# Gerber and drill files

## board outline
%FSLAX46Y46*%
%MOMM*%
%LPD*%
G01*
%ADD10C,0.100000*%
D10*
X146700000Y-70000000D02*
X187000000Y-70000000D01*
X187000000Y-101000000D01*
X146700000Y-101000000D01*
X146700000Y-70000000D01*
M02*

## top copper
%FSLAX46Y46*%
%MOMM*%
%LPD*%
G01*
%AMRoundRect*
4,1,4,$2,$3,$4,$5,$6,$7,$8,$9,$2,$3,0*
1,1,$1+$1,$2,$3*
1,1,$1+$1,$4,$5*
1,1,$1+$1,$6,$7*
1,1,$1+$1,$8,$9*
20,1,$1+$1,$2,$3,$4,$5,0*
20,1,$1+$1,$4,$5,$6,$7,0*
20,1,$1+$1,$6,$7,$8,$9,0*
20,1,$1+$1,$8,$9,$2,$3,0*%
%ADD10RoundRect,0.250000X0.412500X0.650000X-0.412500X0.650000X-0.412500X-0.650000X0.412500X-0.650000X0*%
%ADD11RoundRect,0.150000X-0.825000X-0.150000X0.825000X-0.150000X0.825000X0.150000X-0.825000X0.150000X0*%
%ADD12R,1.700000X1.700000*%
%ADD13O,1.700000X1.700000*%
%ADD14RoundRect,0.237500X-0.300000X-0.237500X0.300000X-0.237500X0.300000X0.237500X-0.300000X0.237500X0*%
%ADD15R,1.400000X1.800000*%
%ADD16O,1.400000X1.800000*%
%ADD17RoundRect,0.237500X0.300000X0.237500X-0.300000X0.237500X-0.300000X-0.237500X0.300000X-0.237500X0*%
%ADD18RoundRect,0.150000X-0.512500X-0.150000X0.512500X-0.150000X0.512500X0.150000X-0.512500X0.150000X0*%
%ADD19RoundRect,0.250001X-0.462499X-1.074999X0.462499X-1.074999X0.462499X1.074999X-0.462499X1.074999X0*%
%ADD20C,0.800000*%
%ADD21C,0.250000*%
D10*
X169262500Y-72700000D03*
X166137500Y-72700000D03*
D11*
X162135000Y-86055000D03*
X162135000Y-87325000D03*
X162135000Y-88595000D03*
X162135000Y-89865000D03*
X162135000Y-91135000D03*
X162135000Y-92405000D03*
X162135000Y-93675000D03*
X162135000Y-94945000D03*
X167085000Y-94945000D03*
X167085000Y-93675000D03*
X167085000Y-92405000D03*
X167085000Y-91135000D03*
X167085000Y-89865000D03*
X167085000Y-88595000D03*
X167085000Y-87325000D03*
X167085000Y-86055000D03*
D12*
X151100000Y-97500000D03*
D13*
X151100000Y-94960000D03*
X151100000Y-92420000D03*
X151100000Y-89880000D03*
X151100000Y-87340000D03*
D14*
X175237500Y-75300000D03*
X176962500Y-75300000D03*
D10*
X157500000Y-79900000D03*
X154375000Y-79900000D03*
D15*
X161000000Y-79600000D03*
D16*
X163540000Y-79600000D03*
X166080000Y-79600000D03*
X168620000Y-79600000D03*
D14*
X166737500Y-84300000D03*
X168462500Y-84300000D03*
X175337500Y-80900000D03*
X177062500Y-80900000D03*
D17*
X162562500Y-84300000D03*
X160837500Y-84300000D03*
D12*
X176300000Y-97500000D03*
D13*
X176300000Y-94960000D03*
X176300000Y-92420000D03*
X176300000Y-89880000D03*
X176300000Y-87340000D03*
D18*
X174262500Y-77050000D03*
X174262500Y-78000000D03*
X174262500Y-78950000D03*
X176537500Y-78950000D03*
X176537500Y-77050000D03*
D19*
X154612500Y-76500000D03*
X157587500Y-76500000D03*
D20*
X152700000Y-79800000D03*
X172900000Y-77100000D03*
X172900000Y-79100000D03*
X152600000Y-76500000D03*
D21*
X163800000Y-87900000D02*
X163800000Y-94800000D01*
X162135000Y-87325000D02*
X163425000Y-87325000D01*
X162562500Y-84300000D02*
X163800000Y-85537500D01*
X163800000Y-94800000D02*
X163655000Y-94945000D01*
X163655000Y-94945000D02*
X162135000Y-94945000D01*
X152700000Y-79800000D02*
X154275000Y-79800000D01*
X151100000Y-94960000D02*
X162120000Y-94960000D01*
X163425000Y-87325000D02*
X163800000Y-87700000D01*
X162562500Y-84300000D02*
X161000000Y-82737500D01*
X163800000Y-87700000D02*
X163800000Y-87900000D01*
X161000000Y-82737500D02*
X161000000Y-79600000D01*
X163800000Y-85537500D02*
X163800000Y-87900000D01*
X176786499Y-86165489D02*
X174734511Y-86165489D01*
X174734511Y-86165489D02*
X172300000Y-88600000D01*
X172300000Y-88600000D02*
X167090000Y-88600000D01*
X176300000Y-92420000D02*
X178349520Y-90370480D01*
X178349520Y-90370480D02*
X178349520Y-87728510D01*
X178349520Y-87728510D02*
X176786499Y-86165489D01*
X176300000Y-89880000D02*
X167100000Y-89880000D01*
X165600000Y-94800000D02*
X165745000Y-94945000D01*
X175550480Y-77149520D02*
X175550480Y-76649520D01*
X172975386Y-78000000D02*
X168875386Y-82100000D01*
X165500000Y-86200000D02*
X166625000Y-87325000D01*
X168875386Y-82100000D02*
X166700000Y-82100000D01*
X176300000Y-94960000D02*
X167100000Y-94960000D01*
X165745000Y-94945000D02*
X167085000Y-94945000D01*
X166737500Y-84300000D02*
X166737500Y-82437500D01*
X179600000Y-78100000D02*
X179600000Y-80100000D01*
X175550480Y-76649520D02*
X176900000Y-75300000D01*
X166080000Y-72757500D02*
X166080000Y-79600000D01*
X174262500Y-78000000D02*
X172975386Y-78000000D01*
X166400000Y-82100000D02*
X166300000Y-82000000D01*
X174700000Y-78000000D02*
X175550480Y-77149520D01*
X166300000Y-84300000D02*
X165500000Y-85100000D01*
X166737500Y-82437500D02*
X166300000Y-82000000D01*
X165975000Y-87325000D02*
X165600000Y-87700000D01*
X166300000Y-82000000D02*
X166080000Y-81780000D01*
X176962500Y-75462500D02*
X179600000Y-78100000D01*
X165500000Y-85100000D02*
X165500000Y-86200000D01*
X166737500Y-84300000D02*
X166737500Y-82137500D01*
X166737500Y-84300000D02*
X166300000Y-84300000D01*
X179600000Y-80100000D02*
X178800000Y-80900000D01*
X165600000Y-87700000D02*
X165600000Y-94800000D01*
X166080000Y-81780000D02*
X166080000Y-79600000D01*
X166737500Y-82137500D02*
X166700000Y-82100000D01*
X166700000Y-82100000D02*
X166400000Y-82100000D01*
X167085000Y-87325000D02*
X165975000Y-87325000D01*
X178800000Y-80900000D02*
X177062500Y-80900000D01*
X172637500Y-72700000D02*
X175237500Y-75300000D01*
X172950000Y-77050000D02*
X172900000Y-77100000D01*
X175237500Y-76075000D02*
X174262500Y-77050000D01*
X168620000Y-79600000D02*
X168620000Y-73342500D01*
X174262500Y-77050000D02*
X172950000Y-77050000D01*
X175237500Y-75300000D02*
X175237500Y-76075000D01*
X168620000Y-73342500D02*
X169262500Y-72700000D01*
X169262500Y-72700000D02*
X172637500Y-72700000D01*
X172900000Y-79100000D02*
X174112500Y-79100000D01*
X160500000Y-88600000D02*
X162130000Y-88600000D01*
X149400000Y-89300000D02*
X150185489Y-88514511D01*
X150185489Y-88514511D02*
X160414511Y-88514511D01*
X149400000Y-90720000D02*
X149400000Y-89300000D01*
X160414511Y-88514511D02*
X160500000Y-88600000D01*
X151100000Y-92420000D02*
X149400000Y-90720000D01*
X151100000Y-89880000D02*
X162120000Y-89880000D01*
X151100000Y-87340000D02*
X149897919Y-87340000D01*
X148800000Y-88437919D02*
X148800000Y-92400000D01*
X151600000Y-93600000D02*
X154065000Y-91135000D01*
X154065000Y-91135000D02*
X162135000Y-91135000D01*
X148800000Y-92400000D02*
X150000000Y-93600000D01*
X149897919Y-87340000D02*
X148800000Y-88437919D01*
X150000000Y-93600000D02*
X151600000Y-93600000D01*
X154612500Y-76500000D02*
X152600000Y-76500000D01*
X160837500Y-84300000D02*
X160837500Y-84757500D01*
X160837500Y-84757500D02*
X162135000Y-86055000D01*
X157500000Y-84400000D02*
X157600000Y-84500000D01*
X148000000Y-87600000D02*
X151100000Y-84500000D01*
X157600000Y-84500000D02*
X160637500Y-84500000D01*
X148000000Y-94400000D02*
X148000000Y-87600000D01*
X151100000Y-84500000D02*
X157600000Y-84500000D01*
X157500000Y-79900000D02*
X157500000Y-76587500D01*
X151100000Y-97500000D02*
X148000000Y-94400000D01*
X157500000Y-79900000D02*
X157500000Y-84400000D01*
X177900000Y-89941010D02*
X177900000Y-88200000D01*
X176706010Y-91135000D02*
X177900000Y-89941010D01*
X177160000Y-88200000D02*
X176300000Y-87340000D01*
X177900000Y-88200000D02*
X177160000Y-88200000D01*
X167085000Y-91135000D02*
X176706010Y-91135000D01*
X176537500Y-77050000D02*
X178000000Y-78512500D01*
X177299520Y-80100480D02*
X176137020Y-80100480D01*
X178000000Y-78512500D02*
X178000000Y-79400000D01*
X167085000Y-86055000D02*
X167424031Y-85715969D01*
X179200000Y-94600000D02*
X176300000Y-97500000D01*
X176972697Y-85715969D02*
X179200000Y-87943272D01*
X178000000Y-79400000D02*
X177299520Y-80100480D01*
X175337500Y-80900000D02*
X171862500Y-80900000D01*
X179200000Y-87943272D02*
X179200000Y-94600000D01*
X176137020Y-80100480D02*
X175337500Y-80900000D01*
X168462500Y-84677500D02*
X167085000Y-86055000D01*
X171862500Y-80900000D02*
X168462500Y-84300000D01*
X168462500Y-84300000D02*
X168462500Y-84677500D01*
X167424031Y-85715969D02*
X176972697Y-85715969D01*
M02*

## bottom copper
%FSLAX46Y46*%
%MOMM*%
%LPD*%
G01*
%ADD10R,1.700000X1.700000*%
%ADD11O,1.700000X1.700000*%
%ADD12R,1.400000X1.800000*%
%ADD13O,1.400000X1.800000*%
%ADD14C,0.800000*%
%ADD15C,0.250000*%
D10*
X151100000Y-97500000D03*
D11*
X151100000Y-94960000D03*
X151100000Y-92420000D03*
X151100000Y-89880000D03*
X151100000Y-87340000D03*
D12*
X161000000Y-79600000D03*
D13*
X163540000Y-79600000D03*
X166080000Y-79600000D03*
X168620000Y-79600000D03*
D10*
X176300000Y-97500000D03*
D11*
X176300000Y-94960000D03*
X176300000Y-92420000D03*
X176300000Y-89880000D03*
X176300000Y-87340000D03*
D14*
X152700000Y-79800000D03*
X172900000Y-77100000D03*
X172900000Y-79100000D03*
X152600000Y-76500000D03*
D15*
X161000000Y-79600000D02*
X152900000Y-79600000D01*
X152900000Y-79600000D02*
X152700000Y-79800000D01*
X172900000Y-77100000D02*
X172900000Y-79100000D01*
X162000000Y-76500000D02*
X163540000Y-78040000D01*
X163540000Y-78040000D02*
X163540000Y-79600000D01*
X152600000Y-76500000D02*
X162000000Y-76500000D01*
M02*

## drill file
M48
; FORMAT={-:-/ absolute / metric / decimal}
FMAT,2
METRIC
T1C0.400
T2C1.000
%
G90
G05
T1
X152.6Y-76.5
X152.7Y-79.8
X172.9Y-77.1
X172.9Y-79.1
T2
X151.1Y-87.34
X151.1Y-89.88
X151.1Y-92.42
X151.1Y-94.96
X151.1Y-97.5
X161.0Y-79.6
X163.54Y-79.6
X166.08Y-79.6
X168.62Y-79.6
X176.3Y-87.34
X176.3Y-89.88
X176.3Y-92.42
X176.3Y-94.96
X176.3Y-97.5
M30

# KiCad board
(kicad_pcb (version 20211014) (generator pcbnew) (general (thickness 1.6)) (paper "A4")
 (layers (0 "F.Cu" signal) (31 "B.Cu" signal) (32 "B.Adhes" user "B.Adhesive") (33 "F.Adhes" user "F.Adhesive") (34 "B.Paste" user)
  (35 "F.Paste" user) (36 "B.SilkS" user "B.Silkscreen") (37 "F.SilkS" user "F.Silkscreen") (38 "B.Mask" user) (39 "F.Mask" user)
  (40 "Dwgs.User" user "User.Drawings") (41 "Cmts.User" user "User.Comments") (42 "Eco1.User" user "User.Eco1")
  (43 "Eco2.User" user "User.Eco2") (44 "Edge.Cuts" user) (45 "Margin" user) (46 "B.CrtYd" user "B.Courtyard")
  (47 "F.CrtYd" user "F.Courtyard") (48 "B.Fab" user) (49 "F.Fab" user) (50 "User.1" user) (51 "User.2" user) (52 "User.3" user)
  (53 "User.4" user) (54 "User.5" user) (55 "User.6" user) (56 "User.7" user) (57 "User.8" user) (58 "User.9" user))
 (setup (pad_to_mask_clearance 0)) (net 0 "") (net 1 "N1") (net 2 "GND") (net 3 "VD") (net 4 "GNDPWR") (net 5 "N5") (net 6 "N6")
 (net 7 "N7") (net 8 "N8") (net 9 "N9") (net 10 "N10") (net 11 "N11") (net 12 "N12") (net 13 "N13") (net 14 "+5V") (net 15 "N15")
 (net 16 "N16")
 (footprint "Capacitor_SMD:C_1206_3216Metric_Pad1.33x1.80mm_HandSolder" (layer "F.Cu") (at 167.7 72.7 180)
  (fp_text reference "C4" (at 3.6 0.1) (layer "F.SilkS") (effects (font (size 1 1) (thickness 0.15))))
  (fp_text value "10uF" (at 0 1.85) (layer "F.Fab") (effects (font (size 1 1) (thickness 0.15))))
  (pad "1" smd roundrect (at -1.5625 0 180) (size 1.325 1.8) (layers "F.Cu" "F.Paste" "F.Mask") (roundrect_rratio 0.1886792453) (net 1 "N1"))
  (pad "2" smd roundrect (at 1.5625 0 180) (size 1.325 1.8) (layers "F.Cu" "F.Paste" "F.Mask") (roundrect_rratio 0.1886792453) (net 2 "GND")))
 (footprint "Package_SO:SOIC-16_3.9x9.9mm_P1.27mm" (layer "F.Cu") (at 164.61 90.5)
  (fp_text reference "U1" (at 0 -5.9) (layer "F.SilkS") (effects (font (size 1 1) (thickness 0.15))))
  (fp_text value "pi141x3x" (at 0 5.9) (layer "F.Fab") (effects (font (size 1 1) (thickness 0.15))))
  (pad "1" smd roundrect (at -2.475 -4.445) (size 1.95 0.6) (layers "F.Cu" "F.Paste" "F.Mask") (roundrect_rratio 0.25) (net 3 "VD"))
  (pad "2" smd roundrect (at -2.475 -3.175) (size 1.95 0.6) (layers "F.Cu" "F.Paste" "F.Mask") (roundrect_rratio 0.25) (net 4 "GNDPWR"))
  (pad "3" smd roundrect (at -2.475 -1.905) (size 1.95 0.6) (layers "F.Cu" "F.Paste" "F.Mask") (roundrect_rratio 0.25) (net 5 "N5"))
  (pad "4" smd roundrect (at -2.475 -0.635) (size 1.95 0.6) (layers "F.Cu" "F.Paste" "F.Mask") (roundrect_rratio 0.25) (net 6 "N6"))
  (pad "5" smd roundrect (at -2.475 0.635) (size 1.95 0.6) (layers "F.Cu" "F.Paste" "F.Mask") (roundrect_rratio 0.25) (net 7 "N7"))
  (pad "6" smd roundrect (at -2.475 1.905) (size 1.95 0.6) (layers "F.Cu" "F.Paste" "F.Mask") (roundrect_rratio 0.25) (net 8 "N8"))
  (pad "7" smd roundrect (at -2.475 3.175) (size 1.95 0.6) (layers "F.Cu" "F.Paste" "F.Mask") (roundrect_rratio 0.25) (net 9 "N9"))
  (pad "8" smd roundrect (at -2.475 4.445) (size 1.95 0.6) (layers "F.Cu" "F.Paste" "F.Mask") (roundrect_rratio 0.25) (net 4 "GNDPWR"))
  (pad "9" smd roundrect (at 2.475 4.445) (size 1.95 0.6) (layers "F.Cu" "F.Paste" "F.Mask") (roundrect_rratio 0.25) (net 2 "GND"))
  (pad "10" smd roundrect (at 2.475 3.175) (size 1.95 0.6) (layers "F.Cu" "F.Paste" "F.Mask") (roundrect_rratio 0.25) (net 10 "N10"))
  (pad "11" smd roundrect (at 2.475 1.905) (size 1.95 0.6) (layers "F.Cu" "F.Paste" "F.Mask") (roundrect_rratio 0.25) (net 2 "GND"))
  (pad "12" smd roundrect (at 2.475 0.635) (size 1.95 0.6) (layers "F.Cu" "F.Paste" "F.Mask") (roundrect_rratio 0.25) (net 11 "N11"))
  (pad "13" smd roundrect (at 2.475 -0.635) (size 1.95 0.6) (layers "F.Cu" "F.Paste" "F.Mask") (roundrect_rratio 0.25) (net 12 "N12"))
  (pad "14" smd roundrect (at 2.475 -1.905) (size 1.95 0.6) (layers "F.Cu" "F.Paste" "F.Mask") (roundrect_rratio 0.25) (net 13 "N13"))
  (pad "15" smd roundrect (at 2.475 -3.175) (size 1.95 0.6) (layers "F.Cu" "F.Paste" "F.Mask") (roundrect_rratio 0.25) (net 2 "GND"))
  (pad "16" smd roundrect (at 2.475 -4.445) (size 1.95 0.6) (layers "F.Cu" "F.Paste" "F.Mask") (roundrect_rratio 0.25) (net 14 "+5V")))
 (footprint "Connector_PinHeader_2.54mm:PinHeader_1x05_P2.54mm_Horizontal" (layer "F.Cu") (at 151.1 97.5 180)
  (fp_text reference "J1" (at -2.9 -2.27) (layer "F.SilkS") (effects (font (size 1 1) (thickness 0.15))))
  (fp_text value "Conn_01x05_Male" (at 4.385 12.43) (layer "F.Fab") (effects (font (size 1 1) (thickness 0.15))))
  (pad "1" thru_hole rect (at 0 0 180) (size 1.7 1.7) (drill 1) (layers *.Cu *.Mask) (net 3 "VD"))
  (pad "2" thru_hole oval (at 0 2.54 180) (size 1.7 1.7) (drill 1) (layers *.Cu *.Mask) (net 4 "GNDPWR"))
  (pad "3" thru_hole oval (at 0 5.08 180) (size 1.7 1.7) (drill 1) (layers *.Cu *.Mask) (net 5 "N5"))
  (pad "4" thru_hole oval (at 0 7.62 180) (size 1.7 1.7) (drill 1) (layers *.Cu *.Mask) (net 6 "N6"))
  (pad "5" thru_hole oval (at 0 10.16 180) (size 1.7 1.7) (drill 1) (layers *.Cu *.Mask) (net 7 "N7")))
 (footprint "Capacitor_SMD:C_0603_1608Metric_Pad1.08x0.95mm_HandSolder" (layer "F.Cu") (at 176.1 75.3)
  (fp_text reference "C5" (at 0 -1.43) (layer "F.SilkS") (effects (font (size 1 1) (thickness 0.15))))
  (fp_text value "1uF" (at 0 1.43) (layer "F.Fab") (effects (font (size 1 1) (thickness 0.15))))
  (pad "1" smd roundrect (at -0.8625 0) (size 1.075 0.95) (layers "F.Cu" "F.Paste" "F.Mask") (roundrect_rratio 0.25) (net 1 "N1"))
  (pad "2" smd roundrect (at 0.8625 0) (size 1.075 0.95) (layers "F.Cu" "F.Paste" "F.Mask") (roundrect_rratio 0.25) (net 2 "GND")))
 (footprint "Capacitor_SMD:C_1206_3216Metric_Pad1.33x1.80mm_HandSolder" (layer "F.Cu") (at 155.9375 79.9 180)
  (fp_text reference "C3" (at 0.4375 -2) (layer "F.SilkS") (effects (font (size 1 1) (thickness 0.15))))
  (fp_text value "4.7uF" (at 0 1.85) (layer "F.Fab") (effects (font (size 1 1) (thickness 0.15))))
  (pad "1" smd roundrect (at -1.5625 0 180) (size 1.325 1.8) (layers "F.Cu" "F.Paste" "F.Mask") (roundrect_rratio 0.1886792453) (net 3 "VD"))
  (pad "2" smd roundrect (at 1.5625 0 180) (size 1.325 1.8) (layers "F.Cu" "F.Paste" "F.Mask") (roundrect_rratio 0.1886792453)
   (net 4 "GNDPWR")))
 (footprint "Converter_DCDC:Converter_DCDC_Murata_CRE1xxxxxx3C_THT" (layer "F.Cu") (at 161 79.6 90)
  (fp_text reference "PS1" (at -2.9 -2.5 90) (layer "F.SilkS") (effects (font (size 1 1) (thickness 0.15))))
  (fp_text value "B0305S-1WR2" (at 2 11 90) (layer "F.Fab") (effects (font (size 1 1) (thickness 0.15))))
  (pad "1" thru_hole rect (at 0 0) (size 1.4 1.8) (drill 1) (layers *.Cu *.Mask) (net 4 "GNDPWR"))
  (pad "2" thru_hole oval (at 0 2.54) (size 1.4 1.8) (drill 1) (layers *.Cu *.Mask) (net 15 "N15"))
  (pad "3" thru_hole oval (at 0 5.08) (size 1.4 1.8) (drill 1) (layers *.Cu *.Mask) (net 2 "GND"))
  (pad "4" thru_hole oval (at 0 7.62) (size 1.4 1.8) (drill 1) (layers *.Cu *.Mask) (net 1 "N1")))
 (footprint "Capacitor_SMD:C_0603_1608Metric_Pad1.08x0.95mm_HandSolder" (layer "F.Cu") (at 167.6 84.3)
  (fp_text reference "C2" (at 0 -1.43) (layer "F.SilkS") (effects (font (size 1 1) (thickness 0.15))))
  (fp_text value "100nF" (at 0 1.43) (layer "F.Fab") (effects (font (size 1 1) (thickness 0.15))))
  (pad "1" smd roundrect (at -0.8625 0) (size 1.075 0.95) (layers "F.Cu" "F.Paste" "F.Mask") (roundrect_rratio 0.25) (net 2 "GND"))
  (pad "2" smd roundrect (at 0.8625 0) (size 1.075 0.95) (layers "F.Cu" "F.Paste" "F.Mask") (roundrect_rratio 0.25) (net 14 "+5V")))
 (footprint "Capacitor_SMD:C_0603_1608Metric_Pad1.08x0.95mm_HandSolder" (layer "F.Cu") (at 176.2 80.9)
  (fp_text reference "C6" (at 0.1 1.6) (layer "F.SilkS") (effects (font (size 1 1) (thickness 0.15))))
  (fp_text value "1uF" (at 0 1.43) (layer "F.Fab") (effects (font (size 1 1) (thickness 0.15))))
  (pad "1" smd roundrect (at -0.8625 0) (size 1.075 0.95) (layers "F.Cu" "F.Paste" "F.Mask") (roundrect_rratio 0.25) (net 14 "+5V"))
  (pad "2" smd roundrect (at 0.8625 0) (size 1.075 0.95) (layers "F.Cu" "F.Paste" "F.Mask") (roundrect_rratio 0.25) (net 2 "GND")))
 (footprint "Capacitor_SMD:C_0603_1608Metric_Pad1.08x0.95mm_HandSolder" (layer "F.Cu") (at 161.7 84.3 180)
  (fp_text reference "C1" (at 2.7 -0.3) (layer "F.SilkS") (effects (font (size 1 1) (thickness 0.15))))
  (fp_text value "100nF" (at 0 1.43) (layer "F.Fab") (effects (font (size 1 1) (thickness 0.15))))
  (pad "1" smd roundrect (at -0.8625 0 180) (size 1.075 0.95) (layers "F.Cu" "F.Paste" "F.Mask") (roundrect_rratio 0.25) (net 4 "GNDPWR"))
  (pad "2" smd roundrect (at 0.8625 0 180) (size 1.075 0.95) (layers "F.Cu" "F.Paste" "F.Mask") (roundrect_rratio 0.25) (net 3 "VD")))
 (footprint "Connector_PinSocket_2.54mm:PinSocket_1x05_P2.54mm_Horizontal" (layer "F.Cu") (at 176.3 97.5 180)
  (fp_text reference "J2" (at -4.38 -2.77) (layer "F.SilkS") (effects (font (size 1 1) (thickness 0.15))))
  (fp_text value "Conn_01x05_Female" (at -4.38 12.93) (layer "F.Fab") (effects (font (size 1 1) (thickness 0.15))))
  (pad "1" thru_hole rect (at 0 0 180) (size 1.7 1.7) (drill 1) (layers *.Cu *.Mask) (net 14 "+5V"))
  (pad "2" thru_hole oval (at 0 2.54 180) (size 1.7 1.7) (drill 1) (layers *.Cu *.Mask) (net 2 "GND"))
  (pad "3" thru_hole oval (at 0 5.08 180) (size 1.7 1.7) (drill 1) (layers *.Cu *.Mask) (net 13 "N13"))
  (pad "4" thru_hole oval (at 0 7.62 180) (size 1.7 1.7) (drill 1) (layers *.Cu *.Mask) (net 12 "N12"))
  (pad "5" thru_hole oval (at 0 10.16 180) (size 1.7 1.7) (drill 1) (layers *.Cu *.Mask) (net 11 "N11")))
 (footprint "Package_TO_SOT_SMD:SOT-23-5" (layer "F.Cu") (at 175.4 78)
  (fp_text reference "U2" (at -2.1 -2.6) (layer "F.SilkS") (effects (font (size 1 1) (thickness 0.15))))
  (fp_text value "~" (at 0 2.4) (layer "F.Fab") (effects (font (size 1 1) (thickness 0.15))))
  (pad "1" smd roundrect (at -1.1375 -0.95) (size 1.325 0.6) (layers "F.Cu" "F.Paste" "F.Mask") (roundrect_rratio 0.25) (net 1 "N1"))
  (pad "2" smd roundrect (at -1.1375 0) (size 1.325 0.6) (layers "F.Cu" "F.Paste" "F.Mask") (roundrect_rratio 0.25) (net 2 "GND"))
  (pad "3" smd roundrect (at -1.1375 0.95) (size 1.325 0.6) (layers "F.Cu" "F.Paste" "F.Mask") (roundrect_rratio 0.25) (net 1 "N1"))
  (pad "4" smd roundrect (at 1.1375 0.95) (size 1.325 0.6) (layers "F.Cu" "F.Paste" "F.Mask") (roundrect_rratio 0.25) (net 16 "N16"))
  (pad "5" smd roundrect (at 1.1375 -0.95) (size 1.325 0.6) (layers "F.Cu" "F.Paste" "F.Mask") (roundrect_rratio 0.25) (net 14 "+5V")))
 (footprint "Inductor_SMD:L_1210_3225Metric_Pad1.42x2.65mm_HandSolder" (layer "F.Cu") (at 156.1 76.5)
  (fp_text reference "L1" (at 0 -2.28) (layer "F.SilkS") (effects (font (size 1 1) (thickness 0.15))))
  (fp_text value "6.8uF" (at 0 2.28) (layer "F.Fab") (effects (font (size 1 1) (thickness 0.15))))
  (pad "1" smd roundrect (at -1.4875 0) (size 1.425 2.65) (layers "F.Cu" "F.Paste" "F.Mask") (roundrect_rratio 0.1754392982) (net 15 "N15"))
  (pad "2" smd roundrect (at 1.4875 0) (size 1.425 2.65) (layers "F.Cu" "F.Paste" "F.Mask") (roundrect_rratio 0.1754392982) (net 3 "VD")))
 (gr_rect (start 187 70) (end 146.7 101) (layer "Edge.Cuts") (width 0.1) (fill none))
 (segment (start 163.8 87.9) (end 163.8 94.8) (width 0.25) (layer "F.Cu") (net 4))
 (segment (start 162.135 87.325) (end 163.425 87.325) (width 0.25) (layer "F.Cu") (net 4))
 (segment (start 162.5625 84.3) (end 163.8 85.5375) (width 0.25) (layer "F.Cu") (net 4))
 (segment (start 163.8 94.8) (end 163.655 94.945) (width 0.25) (layer "F.Cu") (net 4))
 (segment (start 163.655 94.945) (end 162.135 94.945) (width 0.25) (layer "F.Cu") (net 4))
 (segment (start 152.7 79.8) (end 154.275 79.8) (width 0.25) (layer "F.Cu") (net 4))
 (segment (start 151.1 94.96) (end 162.12 94.96) (width 0.25) (layer "F.Cu") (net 4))
 (segment (start 163.425 87.325) (end 163.8 87.7) (width 0.25) (layer "F.Cu") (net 4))
 (segment (start 162.5625 84.3) (end 161 82.7375) (width 0.25) (layer "F.Cu") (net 4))
 (segment (start 163.8 87.7) (end 163.8 87.9) (width 0.25) (layer "F.Cu") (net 4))
 (segment (start 161 82.7375) (end 161 79.6) (width 0.25) (layer "F.Cu") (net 4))
 (segment (start 163.8 85.5375) (end 163.8 87.9) (width 0.25) (layer "F.Cu") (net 4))
 (via (at 152.7 79.8) (size 0.8) (drill 0.4) (layers "F.Cu" "B.Cu") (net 4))
 (segment (start 161 79.6) (end 152.9 79.6) (width 0.25) (layer "B.Cu") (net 4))
 (segment (start 152.9 79.6) (end 152.7 79.8) (width 0.25) (layer "B.Cu") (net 4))
 (segment (start 176.786499 86.165489) (end 174.734511 86.165489) (width 0.25) (layer "F.Cu") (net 13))
 (segment (start 174.734511 86.165489) (end 172.3 88.6) (width 0.25) (layer "F.Cu") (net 13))
 (segment (start 172.3 88.6) (end 167.09 88.6) (width 0.25) (layer "F.Cu") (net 13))
 (segment (start 176.3 92.42) (end 178.34952 90.37048) (width 0.25) (layer "F.Cu") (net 13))
 (segment (start 178.34952 90.37048) (end 178.34952 87.72851) (width 0.25) (layer "F.Cu") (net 13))
 (segment (start 178.34952 87.72851) (end 176.786499 86.165489) (width 0.25) (layer "F.Cu") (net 13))
 (segment (start 176.3 89.88) (end 167.1 89.88) (width 0.25) (layer "F.Cu") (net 12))
 (segment (start 165.6 94.8) (end 165.745 94.945) (width 0.25) (layer "F.Cu") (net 2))
 (segment (start 175.55048 77.14952) (end 175.55048 76.64952) (width 0.25) (layer "F.Cu") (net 2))
 (segment (start 172.975386 78) (end 168.875386 82.1) (width 0.25) (layer "F.Cu") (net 2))
 (segment (start 165.5 86.2) (end 166.625 87.325) (width 0.25) (layer "F.Cu") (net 2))
 (segment (start 168.875386 82.1) (end 166.7 82.1) (width 0.25) (layer "F.Cu") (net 2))
 (segment (start 176.3 94.96) (end 167.1 94.96) (width 0.25) (layer "F.Cu") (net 2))
 (segment (start 165.745 94.945) (end 167.085 94.945) (width 0.25) (layer "F.Cu") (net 2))
 (segment (start 166.7375 84.3) (end 166.7375 82.4375) (width 0.25) (layer "F.Cu") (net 2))
 (segment (start 179.6 78.1) (end 179.6 80.1) (width 0.25) (layer "F.Cu") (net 2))
 (segment (start 175.55048 76.64952) (end 176.9 75.3) (width 0.25) (layer "F.Cu") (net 2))
 (segment (start 166.08 72.7575) (end 166.08 79.6) (width 0.25) (layer "F.Cu") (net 2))
 (segment (start 174.2625 78) (end 172.975386 78) (width 0.25) (layer "F.Cu") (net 2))
 (segment (start 166.4 82.1) (end 166.3 82) (width 0.25) (layer "F.Cu") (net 2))
 (segment (start 174.7 78) (end 175.55048 77.14952) (width 0.25) (layer "F.Cu") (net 2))
 (segment (start 166.3 84.3) (end 165.5 85.1) (width 0.25) (layer "F.Cu") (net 2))
 (segment (start 166.7375 82.4375) (end 166.3 82) (width 0.25) (layer "F.Cu") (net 2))
 (segment (start 165.975 87.325) (end 165.6 87.7) (width 0.25) (layer "F.Cu") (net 2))
 (segment (start 166.3 82) (end 166.08 81.78) (width 0.25) (layer "F.Cu") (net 2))
 (segment (start 176.9625 75.4625) (end 179.6 78.1) (width 0.25) (layer "F.Cu") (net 2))
 (segment (start 165.5 85.1) (end 165.5 86.2) (width 0.25) (layer "F.Cu") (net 2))
 (segment (start 166.7375 84.3) (end 166.7375 82.1375) (width 0.25) (layer "F.Cu") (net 2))
 (segment (start 166.7375 84.3) (end 166.3 84.3) (width 0.25) (layer "F.Cu") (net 2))
 (segment (start 179.6 80.1) (end 178.8 80.9) (width 0.25) (layer "F.Cu") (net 2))
 (segment (start 165.6 87.7) (end 165.6 94.8) (width 0.25) (layer "F.Cu") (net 2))
 (segment (start 166.08 81.78) (end 166.08 79.6) (width 0.25) (layer "F.Cu") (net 2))
 (segment (start 166.7375 82.1375) (end 166.7 82.1) (width 0.25) (layer "F.Cu") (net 2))
 (segment (start 166.7 82.1) (end 166.4 82.1) (width 0.25) (layer "F.Cu") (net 2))
 (segment (start 167.085 87.325) (end 165.975 87.325) (width 0.25) (layer "F.Cu") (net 2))
 (segment (start 178.8 80.9) (end 177.0625 80.9) (width 0.25) (layer "F.Cu") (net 2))
 (segment (start 172.6375 72.7) (end 175.2375 75.3) (width 0.25) (layer "F.Cu") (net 1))
 (segment (start 172.95 77.05) (end 172.9 77.1) (width 0.25) (layer "F.Cu") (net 1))
 (segment (start 175.2375 76.075) (end 174.2625 77.05) (width 0.25) (layer "F.Cu") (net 1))
 (segment (start 168.62 79.6) (end 168.62 73.3425) (width 0.25) (layer "F.Cu") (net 1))
 (segment (start 174.2625 77.05) (end 172.95 77.05) (width 0.25) (layer "F.Cu") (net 1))
 (segment (start 175.2375 75.3) (end 175.2375 76.075) (width 0.25) (layer "F.Cu") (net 1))
 (segment (start 168.62 73.3425) (end 169.2625 72.7) (width 0.25) (layer "F.Cu") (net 1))
 (segment (start 169.2625 72.7) (end 172.6375 72.7) (width 0.25) (layer "F.Cu") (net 1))
 (segment (start 172.9 79.1) (end 174.1125 79.1) (width 0.25) (layer "F.Cu") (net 1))
 (via (at 172.9 77.1) (size 0.8) (drill 0.4) (layers "F.Cu" "B.Cu") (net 1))
 (via (at 172.9 79.1) (size 0.8) (drill 0.4) (layers "F.Cu" "B.Cu") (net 1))
 (segment (start 172.9 77.1) (end 172.9 79.1) (width 0.25) (layer "B.Cu") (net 1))
 (segment (start 160.5 88.6) (end 162.13 88.6) (width 0.25) (layer "F.Cu") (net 5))
 (segment (start 149.4 89.3) (end 150.185489 88.514511) (width 0.25) (layer "F.Cu") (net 5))
 (segment (start 150.185489 88.514511) (end 160.414511 88.514511) (width 0.25) (layer "F.Cu") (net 5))
 (segment (start 149.4 90.72) (end 149.4 89.3) (width 0.25) (layer "F.Cu") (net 5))
 (segment (start 160.414511 88.514511) (end 160.5 88.6) (width 0.25) (layer "F.Cu") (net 5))
 (segment (start 151.1 92.42) (end 149.4 90.72) (width 0.25) (layer "F.Cu") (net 5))
 (segment (start 151.1 89.88) (end 162.12 89.88) (width 0.25) (layer "F.Cu") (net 6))
 (segment (start 151.1 87.34) (end 149.897919 87.34) (width 0.25) (layer "F.Cu") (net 7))
 (segment (start 148.8 88.437919) (end 148.8 92.4) (width 0.25) (layer "F.Cu") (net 7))
 (segment (start 151.6 93.6) (end 154.065 91.135) (width 0.25) (layer "F.Cu") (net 7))
 (segment (start 154.065 91.135) (end 162.135 91.135) (width 0.25) (layer "F.Cu") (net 7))
 (segment (start 148.8 92.4) (end 150 93.6) (width 0.25) (layer "F.Cu") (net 7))
 (segment (start 149.897919 87.34) (end 148.8 88.437919) (width 0.25) (layer "F.Cu") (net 7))
 (segment (start 150 93.6) (end 151.6 93.6) (width 0.25) (layer "F.Cu") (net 7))
 (segment (start 154.6125 76.5) (end 152.6 76.5) (width 0.25) (layer "F.Cu") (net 15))
 (via (at 152.6 76.5) (size 0.8) (drill 0.4) (layers "F.Cu" "B.Cu") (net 15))
 (segment (start 162 76.5) (end 163.54 78.04) (width 0.25) (layer "B.Cu") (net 15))
 (segment (start 163.54 78.04) (end 163.54 79.6) (width 0.25) (layer "B.Cu") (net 15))
 (segment (start 152.6 76.5) (end 162 76.5) (width 0.25) (layer "B.Cu") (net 15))
 (segment (start 160.8375 84.3) (end 160.8375 84.7575) (width 0.25) (layer "F.Cu") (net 3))
 (segment (start 160.8375 84.7575) (end 162.135 86.055) (width 0.25) (layer "F.Cu") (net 3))
 (segment (start 157.5 84.4) (end 157.6 84.5) (width 0.25) (layer "F.Cu") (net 3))
 (segment (start 148 87.6) (end 151.1 84.5) (width 0.25) (layer "F.Cu") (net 3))
 (segment (start 157.6 84.5) (end 160.6375 84.5) (width 0.25) (layer "F.Cu") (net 3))
 (segment (start 148 94.4) (end 148 87.6) (width 0.25) (layer "F.Cu") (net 3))
 (segment (start 151.1 84.5) (end 157.6 84.5) (width 0.25) (layer "F.Cu") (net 3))
 (segment (start 157.5 79.9) (end 157.5 76.5875) (width 0.25) (layer "F.Cu") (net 3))
 (segment (start 151.1 97.5) (end 148 94.4) (width 0.25) (layer "F.Cu") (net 3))
 (segment (start 157.5 79.9) (end 157.5 84.4) (width 0.25) (layer "F.Cu") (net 3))
 (segment (start 177.9 89.94101) (end 177.9 88.2) (width 0.25) (layer "F.Cu") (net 11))
 (segment (start 176.70601 91.135) (end 177.9 89.94101) (width 0.25) (layer "F.Cu") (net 11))
 (segment (start 177.16 88.2) (end 176.3 87.34) (width 0.25) (layer "F.Cu") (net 11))
 (segment (start 177.9 88.2) (end 177.16 88.2) (width 0.25) (layer "F.Cu") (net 11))
 (segment (start 167.085 91.135) (end 176.70601 91.135) (width 0.25) (layer "F.Cu") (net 11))
 (segment (start 176.5375 77.05) (end 178 78.5125) (width 0.25) (layer "F.Cu") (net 14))
 (segment (start 177.29952 80.10048) (end 176.13702 80.10048) (width 0.25) (layer "F.Cu") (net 14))
 (segment (start 178 78.5125) (end 178 79.4) (width 0.25) (layer "F.Cu") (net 14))
 (segment (start 167.085 86.055) (end 167.424031 85.715969) (width 0.25) (layer "F.Cu") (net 14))
 (segment (start 179.2 94.6) (end 176.3 97.5) (width 0.25) (layer "F.Cu") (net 14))
 (segment (start 176.972697 85.715969) (end 179.2 87.943272) (width 0.25) (layer "F.Cu") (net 14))
 (segment (start 178 79.4) (end 177.29952 80.10048) (width 0.25) (layer "F.Cu") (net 14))
 (segment (start 175.3375 80.9) (end 171.8625 80.9) (width 0.25) (layer "F.Cu") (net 14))
 (segment (start 179.2 87.943272) (end 179.2 94.6) (width 0.25) (layer "F.Cu") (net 14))
 (segment (start 176.13702 80.10048) (end 175.3375 80.9) (width 0.25) (layer "F.Cu") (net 14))
 (segment (start 168.4625 84.6775) (end 167.085 86.055) (width 0.25) (layer "F.Cu") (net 14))
 (segment (start 171.8625 80.9) (end 168.4625 84.3) (width 0.25) (layer "F.Cu") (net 14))
 (segment (start 168.4625 84.3) (end 168.4625 84.6775) (width 0.25) (layer "F.Cu") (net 14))
 (segment (start 167.424031 85.715969) (end 176.972697 85.715969) (width 0.25) (layer "F.Cu") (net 14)))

